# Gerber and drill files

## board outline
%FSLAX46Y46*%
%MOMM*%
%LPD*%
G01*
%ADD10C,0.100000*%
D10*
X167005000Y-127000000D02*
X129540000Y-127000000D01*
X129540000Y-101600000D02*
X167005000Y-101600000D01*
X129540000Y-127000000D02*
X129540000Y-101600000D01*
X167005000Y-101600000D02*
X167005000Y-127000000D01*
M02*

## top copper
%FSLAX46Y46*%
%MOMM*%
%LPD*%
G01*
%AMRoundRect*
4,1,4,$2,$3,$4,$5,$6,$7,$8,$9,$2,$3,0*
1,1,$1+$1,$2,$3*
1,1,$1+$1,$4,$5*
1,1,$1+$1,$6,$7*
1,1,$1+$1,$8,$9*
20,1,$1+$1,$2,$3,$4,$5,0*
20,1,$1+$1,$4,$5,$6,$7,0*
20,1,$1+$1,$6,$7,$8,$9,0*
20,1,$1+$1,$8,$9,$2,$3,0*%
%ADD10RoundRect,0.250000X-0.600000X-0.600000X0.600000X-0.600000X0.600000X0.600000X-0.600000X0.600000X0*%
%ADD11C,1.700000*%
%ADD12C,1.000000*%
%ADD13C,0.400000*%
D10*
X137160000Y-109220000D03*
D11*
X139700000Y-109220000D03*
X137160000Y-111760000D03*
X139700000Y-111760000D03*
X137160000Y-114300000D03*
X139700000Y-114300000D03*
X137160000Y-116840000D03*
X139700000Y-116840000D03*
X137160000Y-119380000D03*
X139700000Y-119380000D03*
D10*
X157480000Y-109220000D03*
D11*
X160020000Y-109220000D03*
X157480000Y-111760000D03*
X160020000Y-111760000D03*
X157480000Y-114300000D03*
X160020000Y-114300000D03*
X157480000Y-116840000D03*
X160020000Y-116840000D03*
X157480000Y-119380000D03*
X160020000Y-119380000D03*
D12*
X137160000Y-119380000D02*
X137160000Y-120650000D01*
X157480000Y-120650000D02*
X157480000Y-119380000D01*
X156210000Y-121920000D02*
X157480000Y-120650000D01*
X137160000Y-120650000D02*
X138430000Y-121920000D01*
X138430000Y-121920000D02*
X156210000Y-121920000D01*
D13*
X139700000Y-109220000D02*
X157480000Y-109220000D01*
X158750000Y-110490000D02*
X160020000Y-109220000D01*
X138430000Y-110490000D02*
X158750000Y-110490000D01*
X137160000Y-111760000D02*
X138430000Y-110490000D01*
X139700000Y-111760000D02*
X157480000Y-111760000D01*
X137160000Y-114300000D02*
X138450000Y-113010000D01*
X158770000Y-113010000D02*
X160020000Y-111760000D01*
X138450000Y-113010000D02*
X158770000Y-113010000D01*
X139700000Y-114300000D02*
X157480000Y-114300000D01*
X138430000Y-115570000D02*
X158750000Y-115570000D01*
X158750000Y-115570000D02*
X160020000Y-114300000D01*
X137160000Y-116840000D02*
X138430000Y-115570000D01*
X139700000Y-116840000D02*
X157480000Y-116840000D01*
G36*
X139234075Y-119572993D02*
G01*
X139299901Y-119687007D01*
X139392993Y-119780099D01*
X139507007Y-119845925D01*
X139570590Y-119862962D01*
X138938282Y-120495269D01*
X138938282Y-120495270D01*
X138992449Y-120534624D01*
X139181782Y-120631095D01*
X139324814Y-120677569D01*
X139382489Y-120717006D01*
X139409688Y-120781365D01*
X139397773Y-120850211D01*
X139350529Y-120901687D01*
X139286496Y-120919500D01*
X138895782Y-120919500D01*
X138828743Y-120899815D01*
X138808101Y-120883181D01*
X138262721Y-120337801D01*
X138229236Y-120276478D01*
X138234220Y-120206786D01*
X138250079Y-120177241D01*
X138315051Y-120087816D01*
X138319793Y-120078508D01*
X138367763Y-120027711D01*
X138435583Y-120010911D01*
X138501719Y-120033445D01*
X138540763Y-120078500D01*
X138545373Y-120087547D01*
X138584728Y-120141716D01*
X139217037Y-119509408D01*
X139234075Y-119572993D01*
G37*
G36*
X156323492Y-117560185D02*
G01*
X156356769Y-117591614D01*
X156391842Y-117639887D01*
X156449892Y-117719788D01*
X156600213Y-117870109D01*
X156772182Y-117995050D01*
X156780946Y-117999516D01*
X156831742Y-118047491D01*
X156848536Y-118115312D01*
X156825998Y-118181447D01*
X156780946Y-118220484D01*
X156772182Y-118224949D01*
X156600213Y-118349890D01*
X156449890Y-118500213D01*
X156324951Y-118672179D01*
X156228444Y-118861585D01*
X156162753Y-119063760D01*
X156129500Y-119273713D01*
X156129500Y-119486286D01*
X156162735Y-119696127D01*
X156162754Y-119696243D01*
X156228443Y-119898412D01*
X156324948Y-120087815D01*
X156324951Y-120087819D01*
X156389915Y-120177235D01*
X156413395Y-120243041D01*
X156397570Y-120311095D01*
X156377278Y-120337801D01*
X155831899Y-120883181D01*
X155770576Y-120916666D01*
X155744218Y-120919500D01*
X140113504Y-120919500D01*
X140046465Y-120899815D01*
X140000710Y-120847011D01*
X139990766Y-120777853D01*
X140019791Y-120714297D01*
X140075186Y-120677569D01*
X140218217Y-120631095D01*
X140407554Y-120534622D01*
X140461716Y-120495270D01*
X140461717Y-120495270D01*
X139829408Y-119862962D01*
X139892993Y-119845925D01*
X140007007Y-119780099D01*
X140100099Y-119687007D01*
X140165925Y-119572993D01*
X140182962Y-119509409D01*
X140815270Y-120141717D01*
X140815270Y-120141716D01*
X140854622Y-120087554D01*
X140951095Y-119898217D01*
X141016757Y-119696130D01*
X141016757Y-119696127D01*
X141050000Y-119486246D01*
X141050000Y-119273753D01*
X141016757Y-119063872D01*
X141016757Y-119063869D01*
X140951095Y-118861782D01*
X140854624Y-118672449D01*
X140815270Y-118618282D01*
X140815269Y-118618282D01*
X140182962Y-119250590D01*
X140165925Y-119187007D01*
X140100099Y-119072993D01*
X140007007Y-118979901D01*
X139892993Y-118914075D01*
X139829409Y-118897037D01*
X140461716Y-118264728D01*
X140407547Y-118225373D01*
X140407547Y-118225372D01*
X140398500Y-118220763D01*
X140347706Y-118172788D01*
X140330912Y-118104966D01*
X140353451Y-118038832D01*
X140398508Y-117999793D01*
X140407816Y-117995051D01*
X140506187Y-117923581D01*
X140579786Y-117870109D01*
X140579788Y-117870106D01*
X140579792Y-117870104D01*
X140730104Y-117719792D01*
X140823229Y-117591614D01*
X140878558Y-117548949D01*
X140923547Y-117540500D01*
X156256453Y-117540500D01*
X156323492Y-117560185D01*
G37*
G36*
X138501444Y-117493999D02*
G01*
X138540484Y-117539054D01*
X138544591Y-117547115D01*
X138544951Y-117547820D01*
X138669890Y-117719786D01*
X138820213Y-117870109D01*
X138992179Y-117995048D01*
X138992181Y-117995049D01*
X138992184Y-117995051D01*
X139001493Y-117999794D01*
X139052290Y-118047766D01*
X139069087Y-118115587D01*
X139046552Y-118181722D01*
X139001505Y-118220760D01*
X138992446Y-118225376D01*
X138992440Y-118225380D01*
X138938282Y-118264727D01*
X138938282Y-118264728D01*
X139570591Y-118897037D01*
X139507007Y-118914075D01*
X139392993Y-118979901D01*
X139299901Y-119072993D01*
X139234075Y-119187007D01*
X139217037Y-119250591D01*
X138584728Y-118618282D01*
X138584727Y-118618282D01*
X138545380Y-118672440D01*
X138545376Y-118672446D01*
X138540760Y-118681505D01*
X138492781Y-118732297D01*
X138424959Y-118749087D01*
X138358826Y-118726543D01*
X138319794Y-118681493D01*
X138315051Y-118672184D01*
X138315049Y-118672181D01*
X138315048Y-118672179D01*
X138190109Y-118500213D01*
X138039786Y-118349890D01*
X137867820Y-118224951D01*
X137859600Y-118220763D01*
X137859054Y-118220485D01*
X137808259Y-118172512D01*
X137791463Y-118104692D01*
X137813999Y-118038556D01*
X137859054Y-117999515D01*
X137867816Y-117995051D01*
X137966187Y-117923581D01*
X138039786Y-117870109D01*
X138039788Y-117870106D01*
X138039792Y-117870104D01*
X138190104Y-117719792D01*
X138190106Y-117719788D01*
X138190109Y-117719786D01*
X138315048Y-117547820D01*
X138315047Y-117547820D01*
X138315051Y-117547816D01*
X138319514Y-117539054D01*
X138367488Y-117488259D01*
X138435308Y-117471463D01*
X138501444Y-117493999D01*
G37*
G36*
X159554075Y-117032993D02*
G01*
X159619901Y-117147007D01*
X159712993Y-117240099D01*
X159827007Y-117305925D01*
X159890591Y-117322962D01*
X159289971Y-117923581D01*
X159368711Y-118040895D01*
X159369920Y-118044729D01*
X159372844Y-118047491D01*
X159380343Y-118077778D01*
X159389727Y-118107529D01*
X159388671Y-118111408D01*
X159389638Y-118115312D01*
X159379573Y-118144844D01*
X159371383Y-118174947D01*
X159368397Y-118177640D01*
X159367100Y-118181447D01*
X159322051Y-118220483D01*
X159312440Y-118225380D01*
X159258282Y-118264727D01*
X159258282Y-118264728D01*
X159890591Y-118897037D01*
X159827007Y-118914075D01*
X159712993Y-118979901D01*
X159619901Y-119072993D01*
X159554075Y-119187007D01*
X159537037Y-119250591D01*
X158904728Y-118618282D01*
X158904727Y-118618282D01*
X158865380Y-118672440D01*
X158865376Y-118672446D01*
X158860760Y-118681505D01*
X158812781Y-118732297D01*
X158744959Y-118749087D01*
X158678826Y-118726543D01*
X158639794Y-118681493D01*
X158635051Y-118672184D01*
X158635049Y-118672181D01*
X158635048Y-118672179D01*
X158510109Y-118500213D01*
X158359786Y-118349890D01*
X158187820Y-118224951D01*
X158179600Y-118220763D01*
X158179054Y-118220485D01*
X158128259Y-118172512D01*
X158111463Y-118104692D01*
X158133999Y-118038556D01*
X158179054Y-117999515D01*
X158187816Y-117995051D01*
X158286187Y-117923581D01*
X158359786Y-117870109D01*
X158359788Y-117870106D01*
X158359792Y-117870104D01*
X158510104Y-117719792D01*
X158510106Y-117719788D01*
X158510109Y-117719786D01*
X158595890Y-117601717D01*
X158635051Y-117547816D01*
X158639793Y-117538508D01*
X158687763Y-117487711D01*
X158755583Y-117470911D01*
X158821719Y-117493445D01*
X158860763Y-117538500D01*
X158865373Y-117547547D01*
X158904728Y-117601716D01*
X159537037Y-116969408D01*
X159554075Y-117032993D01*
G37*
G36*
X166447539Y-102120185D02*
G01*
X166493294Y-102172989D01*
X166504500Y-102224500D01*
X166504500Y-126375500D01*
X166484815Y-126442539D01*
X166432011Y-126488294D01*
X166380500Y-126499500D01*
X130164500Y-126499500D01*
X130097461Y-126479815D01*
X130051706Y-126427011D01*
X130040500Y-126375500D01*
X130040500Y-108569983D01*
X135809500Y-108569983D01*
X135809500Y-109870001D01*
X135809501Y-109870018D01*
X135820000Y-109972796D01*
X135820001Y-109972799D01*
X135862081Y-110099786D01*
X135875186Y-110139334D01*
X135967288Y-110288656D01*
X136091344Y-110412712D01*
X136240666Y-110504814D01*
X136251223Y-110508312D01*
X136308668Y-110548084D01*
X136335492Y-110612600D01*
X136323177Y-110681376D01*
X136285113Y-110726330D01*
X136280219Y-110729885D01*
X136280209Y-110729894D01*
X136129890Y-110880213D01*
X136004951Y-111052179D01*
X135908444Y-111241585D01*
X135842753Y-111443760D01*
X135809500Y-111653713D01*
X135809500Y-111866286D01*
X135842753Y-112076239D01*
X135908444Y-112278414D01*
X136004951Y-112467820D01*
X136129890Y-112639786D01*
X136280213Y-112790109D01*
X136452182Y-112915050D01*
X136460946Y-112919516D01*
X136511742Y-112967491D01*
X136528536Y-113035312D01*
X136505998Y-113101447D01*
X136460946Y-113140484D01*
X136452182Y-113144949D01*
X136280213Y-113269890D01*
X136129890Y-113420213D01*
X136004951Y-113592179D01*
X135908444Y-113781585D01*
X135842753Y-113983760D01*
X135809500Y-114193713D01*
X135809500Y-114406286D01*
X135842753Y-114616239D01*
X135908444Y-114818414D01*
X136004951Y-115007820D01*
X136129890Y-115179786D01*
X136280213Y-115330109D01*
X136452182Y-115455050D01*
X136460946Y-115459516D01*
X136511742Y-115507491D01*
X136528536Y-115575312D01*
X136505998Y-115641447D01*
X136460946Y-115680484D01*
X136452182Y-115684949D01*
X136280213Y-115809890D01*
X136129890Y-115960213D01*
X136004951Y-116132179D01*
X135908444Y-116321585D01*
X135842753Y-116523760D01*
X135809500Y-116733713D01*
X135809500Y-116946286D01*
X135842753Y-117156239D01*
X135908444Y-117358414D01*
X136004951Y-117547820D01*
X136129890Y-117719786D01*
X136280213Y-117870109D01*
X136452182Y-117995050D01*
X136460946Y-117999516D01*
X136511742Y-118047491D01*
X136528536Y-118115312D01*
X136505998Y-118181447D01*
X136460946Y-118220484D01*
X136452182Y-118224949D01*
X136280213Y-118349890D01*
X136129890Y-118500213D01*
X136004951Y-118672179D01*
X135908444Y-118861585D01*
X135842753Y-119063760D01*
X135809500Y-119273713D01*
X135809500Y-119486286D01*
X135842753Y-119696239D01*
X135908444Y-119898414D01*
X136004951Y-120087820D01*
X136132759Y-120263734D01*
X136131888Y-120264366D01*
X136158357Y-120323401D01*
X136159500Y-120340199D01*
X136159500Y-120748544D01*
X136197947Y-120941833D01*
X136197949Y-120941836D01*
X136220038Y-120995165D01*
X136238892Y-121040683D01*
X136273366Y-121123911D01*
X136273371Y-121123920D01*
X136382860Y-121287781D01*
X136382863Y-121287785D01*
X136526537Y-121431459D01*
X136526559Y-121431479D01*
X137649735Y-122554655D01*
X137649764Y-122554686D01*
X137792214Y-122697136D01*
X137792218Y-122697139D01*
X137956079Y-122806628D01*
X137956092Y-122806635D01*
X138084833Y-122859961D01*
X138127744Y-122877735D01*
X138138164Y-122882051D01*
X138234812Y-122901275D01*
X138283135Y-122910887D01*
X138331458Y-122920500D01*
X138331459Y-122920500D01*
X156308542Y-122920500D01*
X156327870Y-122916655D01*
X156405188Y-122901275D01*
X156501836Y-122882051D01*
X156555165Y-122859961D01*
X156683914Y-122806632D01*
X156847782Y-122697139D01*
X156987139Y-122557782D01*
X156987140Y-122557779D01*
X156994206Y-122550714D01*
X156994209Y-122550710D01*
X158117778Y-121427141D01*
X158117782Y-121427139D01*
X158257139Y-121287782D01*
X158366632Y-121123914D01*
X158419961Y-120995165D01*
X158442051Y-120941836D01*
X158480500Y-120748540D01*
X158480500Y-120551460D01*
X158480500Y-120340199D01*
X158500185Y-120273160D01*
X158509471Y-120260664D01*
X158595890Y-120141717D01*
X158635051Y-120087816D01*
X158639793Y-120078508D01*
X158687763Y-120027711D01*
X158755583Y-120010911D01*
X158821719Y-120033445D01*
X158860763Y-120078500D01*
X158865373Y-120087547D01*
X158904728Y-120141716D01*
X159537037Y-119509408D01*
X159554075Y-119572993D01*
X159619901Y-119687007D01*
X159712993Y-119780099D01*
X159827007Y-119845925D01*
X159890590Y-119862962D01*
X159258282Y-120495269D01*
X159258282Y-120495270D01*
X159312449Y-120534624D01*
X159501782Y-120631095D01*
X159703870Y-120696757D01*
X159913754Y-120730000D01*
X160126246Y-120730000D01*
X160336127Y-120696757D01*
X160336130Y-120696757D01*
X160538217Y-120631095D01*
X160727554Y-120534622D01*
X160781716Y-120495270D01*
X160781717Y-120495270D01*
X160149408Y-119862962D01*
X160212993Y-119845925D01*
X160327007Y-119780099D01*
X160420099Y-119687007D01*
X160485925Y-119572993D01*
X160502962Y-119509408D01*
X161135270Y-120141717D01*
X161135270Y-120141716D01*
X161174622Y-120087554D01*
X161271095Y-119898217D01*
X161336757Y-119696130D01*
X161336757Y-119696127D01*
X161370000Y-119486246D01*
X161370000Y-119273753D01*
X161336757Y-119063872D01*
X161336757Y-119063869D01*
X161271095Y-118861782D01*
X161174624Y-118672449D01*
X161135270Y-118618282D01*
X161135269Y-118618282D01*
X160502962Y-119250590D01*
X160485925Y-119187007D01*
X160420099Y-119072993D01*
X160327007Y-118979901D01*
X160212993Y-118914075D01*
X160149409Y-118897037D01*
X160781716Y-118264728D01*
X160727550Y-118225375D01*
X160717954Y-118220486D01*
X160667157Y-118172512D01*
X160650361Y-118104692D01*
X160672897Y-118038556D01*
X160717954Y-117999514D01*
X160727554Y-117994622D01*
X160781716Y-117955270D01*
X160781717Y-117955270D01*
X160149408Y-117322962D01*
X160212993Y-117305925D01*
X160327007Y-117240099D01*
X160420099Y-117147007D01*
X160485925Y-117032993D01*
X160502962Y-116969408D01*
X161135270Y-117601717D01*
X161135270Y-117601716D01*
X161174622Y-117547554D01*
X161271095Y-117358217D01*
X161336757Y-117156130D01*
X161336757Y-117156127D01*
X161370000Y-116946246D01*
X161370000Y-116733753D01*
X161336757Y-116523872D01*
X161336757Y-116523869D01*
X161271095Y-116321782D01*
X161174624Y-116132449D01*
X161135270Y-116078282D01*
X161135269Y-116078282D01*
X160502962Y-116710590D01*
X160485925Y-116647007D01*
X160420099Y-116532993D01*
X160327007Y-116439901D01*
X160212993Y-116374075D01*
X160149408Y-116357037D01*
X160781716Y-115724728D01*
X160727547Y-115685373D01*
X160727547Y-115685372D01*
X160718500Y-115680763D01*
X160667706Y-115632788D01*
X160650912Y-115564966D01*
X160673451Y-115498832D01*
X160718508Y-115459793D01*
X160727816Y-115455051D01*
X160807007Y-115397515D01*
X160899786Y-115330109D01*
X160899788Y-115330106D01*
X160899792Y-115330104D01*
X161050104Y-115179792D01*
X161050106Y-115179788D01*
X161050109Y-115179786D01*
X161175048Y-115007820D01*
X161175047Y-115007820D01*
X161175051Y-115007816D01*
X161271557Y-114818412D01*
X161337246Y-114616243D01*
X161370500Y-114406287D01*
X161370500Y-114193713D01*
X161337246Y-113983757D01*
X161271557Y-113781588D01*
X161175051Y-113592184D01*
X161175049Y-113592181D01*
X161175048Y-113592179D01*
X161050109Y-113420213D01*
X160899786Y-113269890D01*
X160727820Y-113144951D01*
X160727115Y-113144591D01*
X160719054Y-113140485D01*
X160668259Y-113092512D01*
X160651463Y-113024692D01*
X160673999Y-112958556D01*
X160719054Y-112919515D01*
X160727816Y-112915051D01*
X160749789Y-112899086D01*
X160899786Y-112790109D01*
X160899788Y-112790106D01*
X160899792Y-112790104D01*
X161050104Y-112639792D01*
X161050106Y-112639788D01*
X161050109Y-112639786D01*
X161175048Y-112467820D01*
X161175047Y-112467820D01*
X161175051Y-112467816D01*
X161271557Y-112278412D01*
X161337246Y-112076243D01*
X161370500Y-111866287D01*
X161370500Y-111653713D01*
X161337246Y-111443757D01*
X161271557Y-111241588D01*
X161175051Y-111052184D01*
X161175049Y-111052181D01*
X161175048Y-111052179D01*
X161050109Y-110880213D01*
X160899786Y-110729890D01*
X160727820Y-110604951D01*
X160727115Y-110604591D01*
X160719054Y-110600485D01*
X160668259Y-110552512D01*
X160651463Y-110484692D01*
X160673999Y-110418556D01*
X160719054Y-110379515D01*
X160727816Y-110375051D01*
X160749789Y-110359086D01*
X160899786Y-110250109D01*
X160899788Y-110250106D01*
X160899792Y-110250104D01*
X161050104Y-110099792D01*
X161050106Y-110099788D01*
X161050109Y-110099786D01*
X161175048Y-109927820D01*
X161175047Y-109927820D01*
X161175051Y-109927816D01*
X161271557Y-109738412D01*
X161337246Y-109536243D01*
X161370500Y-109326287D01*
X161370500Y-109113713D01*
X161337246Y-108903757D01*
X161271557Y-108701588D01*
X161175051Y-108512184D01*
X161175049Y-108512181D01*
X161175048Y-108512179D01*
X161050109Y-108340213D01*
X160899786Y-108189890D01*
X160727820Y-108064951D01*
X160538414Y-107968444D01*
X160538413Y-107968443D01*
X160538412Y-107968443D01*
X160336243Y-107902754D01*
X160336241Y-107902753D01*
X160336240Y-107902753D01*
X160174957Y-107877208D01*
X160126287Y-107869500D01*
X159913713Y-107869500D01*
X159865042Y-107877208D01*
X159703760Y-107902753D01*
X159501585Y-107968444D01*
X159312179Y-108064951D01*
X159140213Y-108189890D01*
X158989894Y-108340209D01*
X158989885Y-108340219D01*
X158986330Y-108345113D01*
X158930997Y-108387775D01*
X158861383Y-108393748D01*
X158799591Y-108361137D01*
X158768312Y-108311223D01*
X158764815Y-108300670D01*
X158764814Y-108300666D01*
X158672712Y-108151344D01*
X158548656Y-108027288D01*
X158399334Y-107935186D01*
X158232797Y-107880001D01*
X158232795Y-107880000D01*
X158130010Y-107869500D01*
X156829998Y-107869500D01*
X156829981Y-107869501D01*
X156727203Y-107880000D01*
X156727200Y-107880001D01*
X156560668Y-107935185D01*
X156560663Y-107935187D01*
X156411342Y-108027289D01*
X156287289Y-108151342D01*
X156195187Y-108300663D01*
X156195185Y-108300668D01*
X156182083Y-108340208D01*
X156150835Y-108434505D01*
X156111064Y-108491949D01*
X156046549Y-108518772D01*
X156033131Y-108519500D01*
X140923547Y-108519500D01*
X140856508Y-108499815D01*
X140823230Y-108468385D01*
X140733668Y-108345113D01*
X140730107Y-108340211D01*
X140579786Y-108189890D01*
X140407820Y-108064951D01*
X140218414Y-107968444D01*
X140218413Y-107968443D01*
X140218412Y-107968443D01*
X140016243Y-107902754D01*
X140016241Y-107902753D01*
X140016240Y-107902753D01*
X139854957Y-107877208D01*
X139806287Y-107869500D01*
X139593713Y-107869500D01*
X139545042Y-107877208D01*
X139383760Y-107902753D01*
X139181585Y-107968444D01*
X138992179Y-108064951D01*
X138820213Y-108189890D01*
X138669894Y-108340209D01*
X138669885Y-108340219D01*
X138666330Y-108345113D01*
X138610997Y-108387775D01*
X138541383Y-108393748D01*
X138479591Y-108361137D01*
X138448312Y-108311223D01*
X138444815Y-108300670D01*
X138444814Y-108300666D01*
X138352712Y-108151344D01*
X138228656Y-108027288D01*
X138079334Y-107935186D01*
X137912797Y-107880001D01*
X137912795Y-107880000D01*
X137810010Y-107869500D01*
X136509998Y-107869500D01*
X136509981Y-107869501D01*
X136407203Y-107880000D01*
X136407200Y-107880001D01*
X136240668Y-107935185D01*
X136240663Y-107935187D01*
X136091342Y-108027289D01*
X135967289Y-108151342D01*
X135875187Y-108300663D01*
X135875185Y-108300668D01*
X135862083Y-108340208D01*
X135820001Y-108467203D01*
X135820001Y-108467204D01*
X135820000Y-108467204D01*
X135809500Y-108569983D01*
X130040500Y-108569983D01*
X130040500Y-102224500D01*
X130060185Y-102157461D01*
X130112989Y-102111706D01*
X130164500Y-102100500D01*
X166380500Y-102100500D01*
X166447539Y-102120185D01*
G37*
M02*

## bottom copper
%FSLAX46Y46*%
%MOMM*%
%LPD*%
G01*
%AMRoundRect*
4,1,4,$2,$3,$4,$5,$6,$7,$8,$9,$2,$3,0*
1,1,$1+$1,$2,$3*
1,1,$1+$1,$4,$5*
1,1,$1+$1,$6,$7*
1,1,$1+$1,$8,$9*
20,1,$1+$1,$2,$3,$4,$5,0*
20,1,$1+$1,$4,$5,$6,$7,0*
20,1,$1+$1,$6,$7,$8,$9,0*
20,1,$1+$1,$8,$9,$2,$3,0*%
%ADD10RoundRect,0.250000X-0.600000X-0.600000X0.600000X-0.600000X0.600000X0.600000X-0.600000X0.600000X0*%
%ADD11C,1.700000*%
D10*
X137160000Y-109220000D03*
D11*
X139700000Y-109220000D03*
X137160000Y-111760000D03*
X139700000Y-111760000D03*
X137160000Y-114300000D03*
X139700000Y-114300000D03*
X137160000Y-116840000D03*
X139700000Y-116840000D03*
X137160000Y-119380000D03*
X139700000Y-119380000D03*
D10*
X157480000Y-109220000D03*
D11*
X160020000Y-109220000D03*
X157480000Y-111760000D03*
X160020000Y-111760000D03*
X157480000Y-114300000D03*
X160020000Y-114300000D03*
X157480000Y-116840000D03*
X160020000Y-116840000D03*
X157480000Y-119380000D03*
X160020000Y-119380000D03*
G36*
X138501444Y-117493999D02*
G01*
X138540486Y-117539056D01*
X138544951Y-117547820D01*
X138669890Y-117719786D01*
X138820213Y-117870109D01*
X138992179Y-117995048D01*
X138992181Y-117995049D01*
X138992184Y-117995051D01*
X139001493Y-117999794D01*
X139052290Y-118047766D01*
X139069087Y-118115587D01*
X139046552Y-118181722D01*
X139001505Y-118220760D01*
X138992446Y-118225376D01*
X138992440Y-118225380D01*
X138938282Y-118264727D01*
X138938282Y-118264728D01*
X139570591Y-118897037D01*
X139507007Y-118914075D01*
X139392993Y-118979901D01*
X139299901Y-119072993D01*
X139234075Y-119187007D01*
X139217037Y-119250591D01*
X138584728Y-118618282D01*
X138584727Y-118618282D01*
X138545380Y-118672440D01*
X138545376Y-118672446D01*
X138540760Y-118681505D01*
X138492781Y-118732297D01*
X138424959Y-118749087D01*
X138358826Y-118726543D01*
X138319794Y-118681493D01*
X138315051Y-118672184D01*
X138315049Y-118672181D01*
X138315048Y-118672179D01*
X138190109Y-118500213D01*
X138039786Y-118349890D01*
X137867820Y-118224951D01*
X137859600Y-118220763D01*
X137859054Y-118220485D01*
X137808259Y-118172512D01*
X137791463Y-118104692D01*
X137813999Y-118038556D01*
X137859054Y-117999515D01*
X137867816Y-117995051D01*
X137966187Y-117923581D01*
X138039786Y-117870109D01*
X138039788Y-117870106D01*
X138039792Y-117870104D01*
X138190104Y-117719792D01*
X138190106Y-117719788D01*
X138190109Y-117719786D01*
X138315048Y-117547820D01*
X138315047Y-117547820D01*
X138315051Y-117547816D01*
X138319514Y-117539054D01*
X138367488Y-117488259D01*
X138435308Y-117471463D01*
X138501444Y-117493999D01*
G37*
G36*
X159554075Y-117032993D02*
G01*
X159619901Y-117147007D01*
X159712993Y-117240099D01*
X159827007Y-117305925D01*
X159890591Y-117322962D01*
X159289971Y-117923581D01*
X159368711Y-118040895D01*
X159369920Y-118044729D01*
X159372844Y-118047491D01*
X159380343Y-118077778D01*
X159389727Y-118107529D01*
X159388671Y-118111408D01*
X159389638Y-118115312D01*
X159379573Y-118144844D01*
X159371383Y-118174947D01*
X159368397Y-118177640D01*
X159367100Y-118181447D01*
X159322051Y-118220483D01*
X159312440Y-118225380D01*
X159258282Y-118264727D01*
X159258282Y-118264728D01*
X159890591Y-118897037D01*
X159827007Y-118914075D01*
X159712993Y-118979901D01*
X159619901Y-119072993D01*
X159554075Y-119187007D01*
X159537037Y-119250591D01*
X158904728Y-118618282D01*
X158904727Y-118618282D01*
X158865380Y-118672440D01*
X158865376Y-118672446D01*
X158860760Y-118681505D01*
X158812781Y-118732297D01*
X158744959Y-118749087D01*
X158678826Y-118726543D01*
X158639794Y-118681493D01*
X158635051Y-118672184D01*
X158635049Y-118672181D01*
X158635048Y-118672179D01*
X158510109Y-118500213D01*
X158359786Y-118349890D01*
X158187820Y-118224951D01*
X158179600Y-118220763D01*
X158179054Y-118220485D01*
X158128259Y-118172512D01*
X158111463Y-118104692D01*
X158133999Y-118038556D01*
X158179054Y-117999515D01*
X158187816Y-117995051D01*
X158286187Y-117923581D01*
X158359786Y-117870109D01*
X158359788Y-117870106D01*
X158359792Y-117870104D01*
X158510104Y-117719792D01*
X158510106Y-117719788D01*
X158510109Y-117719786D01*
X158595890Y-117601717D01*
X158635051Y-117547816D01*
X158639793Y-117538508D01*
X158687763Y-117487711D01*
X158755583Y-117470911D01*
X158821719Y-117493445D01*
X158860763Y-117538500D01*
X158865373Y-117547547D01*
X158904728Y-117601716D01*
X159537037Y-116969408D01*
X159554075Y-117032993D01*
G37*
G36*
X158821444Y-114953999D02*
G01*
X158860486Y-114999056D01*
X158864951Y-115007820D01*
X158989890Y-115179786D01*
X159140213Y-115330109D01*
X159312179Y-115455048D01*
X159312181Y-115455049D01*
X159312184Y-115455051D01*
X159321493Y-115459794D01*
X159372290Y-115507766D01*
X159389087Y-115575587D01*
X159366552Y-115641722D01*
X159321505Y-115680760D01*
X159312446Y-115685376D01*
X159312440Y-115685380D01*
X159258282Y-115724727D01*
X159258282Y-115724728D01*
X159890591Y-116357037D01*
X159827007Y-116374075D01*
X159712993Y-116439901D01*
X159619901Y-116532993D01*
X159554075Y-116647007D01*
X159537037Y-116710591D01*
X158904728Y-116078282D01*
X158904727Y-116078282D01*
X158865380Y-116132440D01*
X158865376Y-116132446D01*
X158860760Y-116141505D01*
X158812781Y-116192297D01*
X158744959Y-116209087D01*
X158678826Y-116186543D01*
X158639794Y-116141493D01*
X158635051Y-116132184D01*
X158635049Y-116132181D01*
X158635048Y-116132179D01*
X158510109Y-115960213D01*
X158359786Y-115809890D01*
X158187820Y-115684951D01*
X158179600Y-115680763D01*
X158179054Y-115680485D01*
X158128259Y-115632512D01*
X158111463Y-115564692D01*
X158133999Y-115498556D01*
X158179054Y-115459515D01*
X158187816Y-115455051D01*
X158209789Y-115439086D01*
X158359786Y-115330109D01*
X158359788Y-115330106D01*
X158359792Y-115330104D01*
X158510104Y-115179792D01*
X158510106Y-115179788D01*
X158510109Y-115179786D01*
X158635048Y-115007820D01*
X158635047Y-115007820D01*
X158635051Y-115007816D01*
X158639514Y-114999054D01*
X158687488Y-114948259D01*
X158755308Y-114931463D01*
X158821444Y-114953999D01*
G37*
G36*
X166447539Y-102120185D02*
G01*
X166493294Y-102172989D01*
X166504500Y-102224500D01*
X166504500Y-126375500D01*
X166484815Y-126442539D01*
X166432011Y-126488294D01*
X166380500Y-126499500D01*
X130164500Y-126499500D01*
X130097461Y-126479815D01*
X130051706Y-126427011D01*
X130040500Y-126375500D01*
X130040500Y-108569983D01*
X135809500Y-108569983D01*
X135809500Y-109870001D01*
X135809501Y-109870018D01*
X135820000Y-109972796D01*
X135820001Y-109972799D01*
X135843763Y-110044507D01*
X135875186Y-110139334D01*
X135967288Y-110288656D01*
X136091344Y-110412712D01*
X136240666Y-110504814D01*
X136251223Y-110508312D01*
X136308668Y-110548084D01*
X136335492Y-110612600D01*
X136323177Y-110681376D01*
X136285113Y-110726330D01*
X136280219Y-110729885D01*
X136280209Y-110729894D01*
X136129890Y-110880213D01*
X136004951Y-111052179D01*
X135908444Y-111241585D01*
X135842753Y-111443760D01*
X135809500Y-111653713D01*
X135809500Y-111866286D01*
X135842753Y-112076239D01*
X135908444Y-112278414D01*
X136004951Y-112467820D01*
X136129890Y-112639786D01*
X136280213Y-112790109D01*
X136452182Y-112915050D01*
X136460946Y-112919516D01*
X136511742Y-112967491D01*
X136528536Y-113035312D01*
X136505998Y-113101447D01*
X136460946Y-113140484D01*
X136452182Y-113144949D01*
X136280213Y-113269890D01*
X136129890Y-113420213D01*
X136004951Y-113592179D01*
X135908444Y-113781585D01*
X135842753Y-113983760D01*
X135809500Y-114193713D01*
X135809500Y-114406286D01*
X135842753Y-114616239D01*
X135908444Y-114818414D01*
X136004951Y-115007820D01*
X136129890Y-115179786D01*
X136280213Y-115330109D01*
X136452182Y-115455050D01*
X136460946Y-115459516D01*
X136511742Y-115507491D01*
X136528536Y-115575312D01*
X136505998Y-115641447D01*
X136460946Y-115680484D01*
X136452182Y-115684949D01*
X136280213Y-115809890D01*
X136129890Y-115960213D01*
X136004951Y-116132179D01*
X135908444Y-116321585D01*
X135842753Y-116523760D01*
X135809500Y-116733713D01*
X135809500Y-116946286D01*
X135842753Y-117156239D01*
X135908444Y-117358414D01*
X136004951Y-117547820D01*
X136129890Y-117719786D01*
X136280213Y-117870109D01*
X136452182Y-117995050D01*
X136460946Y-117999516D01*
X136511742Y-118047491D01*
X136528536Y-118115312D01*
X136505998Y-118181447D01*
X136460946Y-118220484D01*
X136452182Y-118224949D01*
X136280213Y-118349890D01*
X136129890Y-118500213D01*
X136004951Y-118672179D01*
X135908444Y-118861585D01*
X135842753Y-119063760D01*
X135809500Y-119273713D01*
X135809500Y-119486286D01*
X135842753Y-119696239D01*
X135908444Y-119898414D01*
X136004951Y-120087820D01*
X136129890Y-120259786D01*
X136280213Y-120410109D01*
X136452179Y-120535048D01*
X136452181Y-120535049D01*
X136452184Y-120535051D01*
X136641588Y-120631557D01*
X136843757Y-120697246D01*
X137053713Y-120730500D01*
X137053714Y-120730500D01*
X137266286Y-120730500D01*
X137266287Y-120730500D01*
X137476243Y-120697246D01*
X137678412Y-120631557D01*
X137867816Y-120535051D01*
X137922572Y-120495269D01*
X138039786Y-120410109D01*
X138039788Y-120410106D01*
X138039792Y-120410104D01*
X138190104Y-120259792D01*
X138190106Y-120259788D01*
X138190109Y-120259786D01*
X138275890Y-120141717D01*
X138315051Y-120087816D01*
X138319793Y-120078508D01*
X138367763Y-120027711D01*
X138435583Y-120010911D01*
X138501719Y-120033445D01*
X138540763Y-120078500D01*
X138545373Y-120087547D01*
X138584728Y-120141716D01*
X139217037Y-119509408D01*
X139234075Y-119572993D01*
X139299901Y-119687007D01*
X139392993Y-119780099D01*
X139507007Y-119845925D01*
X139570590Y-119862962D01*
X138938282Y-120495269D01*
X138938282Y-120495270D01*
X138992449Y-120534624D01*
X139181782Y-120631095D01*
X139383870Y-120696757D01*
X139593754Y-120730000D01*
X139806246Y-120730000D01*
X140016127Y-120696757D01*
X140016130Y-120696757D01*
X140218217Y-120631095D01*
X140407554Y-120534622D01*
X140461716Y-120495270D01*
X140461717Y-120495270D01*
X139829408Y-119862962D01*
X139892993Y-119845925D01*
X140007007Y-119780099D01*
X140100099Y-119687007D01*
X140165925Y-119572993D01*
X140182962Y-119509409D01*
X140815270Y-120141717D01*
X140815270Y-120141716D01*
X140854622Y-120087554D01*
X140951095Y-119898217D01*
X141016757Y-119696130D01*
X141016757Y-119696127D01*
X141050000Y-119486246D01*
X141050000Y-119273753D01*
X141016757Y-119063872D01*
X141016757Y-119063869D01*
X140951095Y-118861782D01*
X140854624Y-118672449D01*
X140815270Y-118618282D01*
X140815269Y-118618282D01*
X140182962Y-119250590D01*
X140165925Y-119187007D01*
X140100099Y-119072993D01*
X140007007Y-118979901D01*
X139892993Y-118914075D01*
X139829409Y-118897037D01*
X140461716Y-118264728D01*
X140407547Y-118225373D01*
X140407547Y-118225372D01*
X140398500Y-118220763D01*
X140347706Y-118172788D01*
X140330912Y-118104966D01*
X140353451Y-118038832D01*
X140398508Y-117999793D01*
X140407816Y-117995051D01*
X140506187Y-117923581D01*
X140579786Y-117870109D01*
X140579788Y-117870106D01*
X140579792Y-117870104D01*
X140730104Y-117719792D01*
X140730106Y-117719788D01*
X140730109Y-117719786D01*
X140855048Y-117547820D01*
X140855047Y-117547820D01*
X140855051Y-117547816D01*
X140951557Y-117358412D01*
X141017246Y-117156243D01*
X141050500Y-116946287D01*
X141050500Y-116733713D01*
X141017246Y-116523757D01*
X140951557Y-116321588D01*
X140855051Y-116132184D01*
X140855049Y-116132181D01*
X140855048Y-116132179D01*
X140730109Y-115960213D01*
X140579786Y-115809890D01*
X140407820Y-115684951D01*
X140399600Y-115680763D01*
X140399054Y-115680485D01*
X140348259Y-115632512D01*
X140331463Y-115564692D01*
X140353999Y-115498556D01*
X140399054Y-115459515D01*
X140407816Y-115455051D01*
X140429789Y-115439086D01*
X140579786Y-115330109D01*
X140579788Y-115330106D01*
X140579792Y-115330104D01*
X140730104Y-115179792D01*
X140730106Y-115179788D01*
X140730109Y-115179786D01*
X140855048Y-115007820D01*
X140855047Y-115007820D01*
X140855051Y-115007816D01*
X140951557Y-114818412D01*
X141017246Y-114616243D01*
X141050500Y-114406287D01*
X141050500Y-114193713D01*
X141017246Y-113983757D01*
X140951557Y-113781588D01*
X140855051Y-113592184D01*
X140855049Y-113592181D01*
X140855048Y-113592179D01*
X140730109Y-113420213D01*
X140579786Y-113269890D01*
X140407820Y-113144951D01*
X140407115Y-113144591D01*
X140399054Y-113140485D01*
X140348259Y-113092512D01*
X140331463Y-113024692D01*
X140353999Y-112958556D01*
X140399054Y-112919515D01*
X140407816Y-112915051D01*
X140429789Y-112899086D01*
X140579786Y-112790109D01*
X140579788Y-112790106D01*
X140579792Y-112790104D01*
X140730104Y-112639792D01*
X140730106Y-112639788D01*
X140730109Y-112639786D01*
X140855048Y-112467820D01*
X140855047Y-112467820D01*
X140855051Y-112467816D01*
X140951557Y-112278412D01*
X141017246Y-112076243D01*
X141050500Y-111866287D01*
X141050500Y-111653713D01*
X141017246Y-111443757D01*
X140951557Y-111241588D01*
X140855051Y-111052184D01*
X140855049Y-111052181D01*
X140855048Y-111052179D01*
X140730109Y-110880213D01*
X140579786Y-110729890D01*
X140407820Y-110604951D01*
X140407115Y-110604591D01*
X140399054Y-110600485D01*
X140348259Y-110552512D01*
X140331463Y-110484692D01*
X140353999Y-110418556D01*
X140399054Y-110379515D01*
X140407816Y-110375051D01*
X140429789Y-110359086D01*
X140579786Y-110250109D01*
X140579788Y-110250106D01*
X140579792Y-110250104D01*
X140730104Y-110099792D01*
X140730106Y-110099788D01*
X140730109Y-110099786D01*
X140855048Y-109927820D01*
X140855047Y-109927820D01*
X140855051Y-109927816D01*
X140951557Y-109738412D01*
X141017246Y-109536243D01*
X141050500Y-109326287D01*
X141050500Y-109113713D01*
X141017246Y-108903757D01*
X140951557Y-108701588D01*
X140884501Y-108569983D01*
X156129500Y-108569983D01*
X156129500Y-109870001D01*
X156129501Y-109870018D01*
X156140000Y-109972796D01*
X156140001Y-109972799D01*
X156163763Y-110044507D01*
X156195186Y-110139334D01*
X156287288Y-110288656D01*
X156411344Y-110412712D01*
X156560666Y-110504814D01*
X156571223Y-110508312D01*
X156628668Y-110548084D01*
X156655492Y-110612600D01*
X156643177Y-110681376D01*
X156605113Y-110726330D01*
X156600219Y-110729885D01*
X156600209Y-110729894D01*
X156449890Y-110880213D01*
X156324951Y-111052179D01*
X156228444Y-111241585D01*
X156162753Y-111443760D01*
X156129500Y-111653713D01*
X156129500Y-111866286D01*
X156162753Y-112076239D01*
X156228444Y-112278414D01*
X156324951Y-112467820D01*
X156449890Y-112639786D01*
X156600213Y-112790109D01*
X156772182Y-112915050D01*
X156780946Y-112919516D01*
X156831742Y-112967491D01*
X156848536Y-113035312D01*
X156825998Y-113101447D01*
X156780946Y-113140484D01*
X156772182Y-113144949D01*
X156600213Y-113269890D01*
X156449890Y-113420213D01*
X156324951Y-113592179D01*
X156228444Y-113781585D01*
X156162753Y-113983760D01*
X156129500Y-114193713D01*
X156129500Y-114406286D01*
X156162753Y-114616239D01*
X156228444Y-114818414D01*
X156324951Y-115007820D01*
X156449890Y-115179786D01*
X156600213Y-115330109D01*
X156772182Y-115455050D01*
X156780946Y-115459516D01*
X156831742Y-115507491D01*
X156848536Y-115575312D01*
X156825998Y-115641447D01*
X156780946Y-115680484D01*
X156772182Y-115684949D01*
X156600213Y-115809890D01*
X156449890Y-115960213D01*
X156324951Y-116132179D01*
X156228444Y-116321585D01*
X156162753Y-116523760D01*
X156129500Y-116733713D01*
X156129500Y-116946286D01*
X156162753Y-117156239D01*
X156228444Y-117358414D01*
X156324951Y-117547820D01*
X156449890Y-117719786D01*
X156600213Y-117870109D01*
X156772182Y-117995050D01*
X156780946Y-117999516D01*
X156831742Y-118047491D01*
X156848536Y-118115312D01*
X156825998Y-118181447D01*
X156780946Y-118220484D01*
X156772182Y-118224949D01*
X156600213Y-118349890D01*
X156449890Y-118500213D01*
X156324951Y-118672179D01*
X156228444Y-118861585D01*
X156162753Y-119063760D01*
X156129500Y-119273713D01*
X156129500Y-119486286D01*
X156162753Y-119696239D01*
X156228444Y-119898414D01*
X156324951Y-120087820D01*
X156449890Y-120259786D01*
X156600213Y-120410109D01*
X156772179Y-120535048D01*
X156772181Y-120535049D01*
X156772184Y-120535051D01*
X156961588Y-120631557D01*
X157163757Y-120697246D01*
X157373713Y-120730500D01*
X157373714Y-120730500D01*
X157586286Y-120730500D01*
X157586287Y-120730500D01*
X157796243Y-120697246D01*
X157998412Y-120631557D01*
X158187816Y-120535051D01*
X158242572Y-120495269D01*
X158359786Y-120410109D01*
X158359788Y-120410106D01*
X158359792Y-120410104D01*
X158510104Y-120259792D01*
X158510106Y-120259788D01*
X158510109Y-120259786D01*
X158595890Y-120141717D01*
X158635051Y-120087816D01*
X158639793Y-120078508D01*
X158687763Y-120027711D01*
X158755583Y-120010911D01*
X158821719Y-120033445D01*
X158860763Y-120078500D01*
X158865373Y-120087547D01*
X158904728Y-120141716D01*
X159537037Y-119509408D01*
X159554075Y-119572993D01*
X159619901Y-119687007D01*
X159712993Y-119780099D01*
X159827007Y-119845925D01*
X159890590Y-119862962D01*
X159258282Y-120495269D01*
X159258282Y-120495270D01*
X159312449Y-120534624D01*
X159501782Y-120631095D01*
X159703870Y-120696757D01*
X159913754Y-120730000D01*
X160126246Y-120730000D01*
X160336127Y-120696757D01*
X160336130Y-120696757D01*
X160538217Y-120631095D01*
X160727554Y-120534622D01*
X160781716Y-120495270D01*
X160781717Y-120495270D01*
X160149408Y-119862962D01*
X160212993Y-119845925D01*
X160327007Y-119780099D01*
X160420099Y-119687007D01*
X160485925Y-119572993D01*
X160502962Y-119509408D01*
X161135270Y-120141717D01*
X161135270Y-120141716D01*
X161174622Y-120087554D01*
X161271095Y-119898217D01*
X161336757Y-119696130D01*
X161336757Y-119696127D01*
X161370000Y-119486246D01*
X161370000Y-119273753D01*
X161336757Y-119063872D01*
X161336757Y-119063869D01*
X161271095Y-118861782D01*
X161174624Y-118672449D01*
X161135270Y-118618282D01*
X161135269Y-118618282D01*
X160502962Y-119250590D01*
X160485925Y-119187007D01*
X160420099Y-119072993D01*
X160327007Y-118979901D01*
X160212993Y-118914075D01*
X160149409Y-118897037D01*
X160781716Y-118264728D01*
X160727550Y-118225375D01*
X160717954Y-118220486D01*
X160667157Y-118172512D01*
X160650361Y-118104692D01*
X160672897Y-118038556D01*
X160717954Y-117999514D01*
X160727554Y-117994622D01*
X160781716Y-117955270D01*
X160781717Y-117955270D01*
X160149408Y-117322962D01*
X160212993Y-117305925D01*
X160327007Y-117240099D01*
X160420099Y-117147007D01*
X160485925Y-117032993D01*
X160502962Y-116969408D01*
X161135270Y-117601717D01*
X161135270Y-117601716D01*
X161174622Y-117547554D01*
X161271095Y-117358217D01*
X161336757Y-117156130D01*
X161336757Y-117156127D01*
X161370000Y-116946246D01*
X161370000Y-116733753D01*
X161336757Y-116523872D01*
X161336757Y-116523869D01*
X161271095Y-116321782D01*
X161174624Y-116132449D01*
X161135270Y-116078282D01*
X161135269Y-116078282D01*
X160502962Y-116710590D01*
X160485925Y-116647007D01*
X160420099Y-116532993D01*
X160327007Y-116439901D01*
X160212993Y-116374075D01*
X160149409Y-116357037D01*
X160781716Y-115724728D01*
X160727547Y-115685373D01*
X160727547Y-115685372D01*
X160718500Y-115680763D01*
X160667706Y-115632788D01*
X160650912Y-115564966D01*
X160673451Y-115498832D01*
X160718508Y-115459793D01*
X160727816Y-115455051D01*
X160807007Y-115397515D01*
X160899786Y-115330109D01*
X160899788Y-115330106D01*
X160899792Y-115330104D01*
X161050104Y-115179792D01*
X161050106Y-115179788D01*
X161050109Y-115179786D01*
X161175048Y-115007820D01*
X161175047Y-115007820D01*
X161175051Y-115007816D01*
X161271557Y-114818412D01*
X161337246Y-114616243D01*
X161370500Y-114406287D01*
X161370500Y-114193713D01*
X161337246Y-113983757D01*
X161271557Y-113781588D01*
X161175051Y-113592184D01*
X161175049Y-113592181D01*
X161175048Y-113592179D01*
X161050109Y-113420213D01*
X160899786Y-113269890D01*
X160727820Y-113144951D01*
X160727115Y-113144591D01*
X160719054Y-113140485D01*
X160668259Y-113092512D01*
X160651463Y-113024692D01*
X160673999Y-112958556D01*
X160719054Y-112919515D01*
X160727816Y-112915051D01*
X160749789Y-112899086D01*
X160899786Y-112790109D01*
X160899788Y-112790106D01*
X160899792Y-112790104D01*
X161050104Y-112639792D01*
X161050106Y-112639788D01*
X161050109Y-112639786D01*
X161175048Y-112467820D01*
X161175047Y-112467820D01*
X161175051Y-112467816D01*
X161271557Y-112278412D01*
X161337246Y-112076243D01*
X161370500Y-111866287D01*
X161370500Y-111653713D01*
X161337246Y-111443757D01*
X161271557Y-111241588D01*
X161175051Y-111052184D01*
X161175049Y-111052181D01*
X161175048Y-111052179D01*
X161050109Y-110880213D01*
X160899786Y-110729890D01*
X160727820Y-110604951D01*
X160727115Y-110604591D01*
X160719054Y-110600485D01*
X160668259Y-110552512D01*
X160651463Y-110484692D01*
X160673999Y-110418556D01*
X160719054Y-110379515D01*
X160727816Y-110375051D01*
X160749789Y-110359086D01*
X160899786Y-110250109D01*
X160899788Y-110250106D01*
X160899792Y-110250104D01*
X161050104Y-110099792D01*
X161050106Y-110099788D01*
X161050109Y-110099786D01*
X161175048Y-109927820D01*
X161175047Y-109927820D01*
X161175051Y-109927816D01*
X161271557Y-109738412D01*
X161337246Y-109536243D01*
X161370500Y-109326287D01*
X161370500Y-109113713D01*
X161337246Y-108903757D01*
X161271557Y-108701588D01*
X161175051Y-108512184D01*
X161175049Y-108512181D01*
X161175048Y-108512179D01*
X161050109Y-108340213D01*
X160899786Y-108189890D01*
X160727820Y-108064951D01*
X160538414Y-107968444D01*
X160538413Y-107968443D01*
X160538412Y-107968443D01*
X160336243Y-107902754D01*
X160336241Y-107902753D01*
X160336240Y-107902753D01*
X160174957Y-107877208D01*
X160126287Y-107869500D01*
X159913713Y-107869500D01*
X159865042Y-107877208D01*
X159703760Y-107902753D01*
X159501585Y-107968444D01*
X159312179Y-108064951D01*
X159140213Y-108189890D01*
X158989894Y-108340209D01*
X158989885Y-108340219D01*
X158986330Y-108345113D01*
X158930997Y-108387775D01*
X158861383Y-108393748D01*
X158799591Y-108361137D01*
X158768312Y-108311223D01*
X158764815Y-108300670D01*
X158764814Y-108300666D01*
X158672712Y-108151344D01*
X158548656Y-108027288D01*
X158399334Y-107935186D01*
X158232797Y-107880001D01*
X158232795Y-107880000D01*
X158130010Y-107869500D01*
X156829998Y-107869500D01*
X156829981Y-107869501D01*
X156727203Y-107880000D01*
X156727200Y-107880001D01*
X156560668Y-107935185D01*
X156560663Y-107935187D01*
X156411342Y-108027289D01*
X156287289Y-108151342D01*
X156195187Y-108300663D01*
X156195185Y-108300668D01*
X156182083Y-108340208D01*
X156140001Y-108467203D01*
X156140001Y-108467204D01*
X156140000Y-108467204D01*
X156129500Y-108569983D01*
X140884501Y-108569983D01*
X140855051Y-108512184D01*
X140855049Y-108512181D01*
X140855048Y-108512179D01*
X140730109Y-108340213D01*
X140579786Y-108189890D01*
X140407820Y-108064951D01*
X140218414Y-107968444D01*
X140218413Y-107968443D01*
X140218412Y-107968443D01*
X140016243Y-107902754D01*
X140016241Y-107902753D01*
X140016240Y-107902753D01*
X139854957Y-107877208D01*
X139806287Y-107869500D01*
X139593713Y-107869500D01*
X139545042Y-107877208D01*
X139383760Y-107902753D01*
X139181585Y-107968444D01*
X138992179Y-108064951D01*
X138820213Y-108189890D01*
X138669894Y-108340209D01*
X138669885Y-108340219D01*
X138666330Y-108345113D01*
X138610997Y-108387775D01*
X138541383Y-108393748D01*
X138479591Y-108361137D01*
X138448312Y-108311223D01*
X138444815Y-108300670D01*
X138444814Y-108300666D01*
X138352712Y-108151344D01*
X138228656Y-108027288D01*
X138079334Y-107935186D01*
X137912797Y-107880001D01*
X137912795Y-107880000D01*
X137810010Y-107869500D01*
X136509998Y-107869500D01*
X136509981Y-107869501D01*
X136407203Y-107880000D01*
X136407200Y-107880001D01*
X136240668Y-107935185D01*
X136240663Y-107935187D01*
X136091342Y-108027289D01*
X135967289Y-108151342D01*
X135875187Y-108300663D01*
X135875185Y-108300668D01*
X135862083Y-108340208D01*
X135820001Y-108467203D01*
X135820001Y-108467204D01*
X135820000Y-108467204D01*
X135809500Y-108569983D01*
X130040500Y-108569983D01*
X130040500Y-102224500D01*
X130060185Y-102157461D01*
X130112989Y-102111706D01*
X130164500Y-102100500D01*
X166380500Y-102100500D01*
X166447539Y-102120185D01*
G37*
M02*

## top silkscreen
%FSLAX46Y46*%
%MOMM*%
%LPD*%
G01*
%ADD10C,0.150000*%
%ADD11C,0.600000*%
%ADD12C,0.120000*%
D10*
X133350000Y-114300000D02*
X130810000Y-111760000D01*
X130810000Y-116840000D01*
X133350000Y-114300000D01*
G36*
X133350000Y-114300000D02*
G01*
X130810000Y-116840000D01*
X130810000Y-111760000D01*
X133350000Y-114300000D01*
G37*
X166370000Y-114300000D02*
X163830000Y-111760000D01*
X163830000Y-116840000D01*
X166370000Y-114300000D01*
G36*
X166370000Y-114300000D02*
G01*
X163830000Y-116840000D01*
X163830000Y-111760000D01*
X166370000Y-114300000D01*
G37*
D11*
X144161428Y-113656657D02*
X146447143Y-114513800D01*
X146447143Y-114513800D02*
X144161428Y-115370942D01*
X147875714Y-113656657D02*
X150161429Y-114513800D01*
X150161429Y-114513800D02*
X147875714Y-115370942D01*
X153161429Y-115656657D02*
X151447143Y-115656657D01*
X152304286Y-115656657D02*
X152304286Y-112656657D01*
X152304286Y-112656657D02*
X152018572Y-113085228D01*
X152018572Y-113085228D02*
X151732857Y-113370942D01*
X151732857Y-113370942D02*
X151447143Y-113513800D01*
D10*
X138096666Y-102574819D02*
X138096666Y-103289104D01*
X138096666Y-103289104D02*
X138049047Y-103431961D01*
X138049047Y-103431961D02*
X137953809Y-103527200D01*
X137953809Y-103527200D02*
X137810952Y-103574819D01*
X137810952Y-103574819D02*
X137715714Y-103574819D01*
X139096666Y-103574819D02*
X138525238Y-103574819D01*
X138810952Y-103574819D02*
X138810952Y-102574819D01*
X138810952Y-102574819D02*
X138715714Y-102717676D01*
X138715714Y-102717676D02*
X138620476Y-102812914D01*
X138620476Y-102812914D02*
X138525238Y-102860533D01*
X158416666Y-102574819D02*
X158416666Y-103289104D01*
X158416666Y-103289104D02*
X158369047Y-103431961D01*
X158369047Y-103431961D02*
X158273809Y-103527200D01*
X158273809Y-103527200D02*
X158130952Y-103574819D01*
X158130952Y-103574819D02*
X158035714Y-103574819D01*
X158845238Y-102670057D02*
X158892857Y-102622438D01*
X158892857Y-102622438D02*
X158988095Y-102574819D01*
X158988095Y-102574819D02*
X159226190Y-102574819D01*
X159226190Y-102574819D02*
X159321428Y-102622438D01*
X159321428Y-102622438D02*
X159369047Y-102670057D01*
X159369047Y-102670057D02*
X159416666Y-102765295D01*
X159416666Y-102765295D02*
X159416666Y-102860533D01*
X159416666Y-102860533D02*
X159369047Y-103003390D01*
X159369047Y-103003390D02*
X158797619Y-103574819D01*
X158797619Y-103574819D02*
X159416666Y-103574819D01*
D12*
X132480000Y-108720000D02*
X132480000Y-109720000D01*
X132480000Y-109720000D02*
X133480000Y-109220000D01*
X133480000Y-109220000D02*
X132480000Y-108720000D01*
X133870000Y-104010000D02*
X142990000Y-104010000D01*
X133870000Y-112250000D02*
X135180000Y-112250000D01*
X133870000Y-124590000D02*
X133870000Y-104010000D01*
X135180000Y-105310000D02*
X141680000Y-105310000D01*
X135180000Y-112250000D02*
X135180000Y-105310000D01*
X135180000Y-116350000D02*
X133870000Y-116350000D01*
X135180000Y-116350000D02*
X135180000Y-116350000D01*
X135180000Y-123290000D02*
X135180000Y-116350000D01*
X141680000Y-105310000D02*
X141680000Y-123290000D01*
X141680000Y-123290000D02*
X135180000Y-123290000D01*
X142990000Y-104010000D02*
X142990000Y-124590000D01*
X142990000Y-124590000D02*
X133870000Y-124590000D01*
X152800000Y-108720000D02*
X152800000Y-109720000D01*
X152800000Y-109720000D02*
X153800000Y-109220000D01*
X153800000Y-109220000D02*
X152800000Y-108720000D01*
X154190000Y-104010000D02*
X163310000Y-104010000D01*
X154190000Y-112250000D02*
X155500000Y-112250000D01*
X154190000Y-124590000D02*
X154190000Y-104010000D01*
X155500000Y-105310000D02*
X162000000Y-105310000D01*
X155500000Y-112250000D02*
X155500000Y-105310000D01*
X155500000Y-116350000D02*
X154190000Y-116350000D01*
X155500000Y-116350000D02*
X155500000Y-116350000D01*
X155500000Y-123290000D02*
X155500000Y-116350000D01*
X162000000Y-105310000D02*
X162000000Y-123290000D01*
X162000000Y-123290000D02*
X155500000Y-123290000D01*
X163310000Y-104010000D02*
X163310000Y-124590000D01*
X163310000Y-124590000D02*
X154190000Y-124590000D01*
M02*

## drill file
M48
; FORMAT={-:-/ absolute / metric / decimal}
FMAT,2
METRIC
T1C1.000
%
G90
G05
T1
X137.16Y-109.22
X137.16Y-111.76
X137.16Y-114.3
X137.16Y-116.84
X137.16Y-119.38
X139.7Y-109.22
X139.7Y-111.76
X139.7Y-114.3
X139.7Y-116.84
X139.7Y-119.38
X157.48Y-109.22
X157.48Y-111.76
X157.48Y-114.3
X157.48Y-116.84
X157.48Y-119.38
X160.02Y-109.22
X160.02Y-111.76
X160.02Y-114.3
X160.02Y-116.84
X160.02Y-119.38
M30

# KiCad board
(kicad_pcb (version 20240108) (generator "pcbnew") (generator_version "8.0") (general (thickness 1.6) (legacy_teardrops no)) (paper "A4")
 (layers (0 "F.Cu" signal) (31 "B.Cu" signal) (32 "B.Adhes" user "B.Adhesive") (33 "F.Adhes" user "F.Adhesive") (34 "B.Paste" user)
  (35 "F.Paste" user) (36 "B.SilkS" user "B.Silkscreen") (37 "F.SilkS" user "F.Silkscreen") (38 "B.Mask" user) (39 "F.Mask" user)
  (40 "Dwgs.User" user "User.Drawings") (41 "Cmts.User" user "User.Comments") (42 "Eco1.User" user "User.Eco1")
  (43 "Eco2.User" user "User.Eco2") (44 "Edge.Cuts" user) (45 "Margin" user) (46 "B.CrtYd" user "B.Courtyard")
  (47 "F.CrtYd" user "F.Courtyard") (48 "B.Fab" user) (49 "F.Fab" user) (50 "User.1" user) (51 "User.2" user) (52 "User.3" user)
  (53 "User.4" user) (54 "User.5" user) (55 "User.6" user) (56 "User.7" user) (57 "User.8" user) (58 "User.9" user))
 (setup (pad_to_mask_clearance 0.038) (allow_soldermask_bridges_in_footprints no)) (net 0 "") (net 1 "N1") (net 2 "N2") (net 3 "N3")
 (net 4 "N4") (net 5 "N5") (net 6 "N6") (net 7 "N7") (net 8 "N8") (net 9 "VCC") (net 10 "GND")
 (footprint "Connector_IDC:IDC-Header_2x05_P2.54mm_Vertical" (layer "F.Cu") (at 137.16 109.22)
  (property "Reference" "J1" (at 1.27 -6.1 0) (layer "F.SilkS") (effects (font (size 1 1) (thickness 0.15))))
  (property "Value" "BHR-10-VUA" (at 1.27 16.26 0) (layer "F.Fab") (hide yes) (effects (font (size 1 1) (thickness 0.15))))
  (fp_line (start -4.68 -0.5) (end -4.68 0.5) (stroke (width 0.12) (type solid)) (layer "F.SilkS"))
  (fp_line (start -4.68 0.5) (end -3.68 0) (stroke (width 0.12) (type solid)) (layer "F.SilkS"))
  (fp_line (start -3.68 0) (end -4.68 -0.5) (stroke (width 0.12) (type solid)) (layer "F.SilkS"))
  (fp_line (start -3.29 -5.21) (end 5.83 -5.21) (stroke (width 0.12) (type solid)) (layer "F.SilkS"))
  (fp_line (start -3.29 3.03) (end -1.98 3.03) (stroke (width 0.12) (type solid)) (layer "F.SilkS"))
  (fp_line (start -3.29 15.37) (end -3.29 -5.21) (stroke (width 0.12) (type solid)) (layer "F.SilkS"))
  (fp_line (start -1.98 -3.91) (end 4.52 -3.91) (stroke (width 0.12) (type solid)) (layer "F.SilkS"))
  (fp_line (start -1.98 3.03) (end -1.98 -3.91) (stroke (width 0.12) (type solid)) (layer "F.SilkS"))
  (fp_line (start -1.98 7.13) (end -3.29 7.13) (stroke (width 0.12) (type solid)) (layer "F.SilkS"))
  (fp_line (start -1.98 7.13) (end -1.98 7.13) (stroke (width 0.12) (type solid)) (layer "F.SilkS"))
  (fp_line (start -1.98 14.07) (end -1.98 7.13) (stroke (width 0.12) (type solid)) (layer "F.SilkS"))
  (fp_line (start 4.52 -3.91) (end 4.52 14.07) (stroke (width 0.12) (type solid)) (layer "F.SilkS"))
  (fp_line (start 4.52 14.07) (end -1.98 14.07) (stroke (width 0.12) (type solid)) (layer "F.SilkS"))
  (fp_line (start 5.83 -5.21) (end 5.83 15.37) (stroke (width 0.12) (type solid)) (layer "F.SilkS"))
  (fp_line (start 5.83 15.37) (end -3.29 15.37) (stroke (width 0.12) (type solid)) (layer "F.SilkS"))
  (pad "1" thru_hole roundrect (at 0 0) (size 1.7 1.7) (drill 1) (layers "*.Cu" "*.Mask") (remove_unused_layers no)
   (roundrect_rratio 0.147059) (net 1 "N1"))
  (pad "2" thru_hole circle (at 2.54 0) (size 1.7 1.7) (drill 1) (layers "*.Cu" "*.Mask") (remove_unused_layers no) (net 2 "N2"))
  (pad "3" thru_hole circle (at 0 2.54) (size 1.7 1.7) (drill 1) (layers "*.Cu" "*.Mask") (remove_unused_layers no) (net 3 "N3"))
  (pad "4" thru_hole circle (at 2.54 2.54) (size 1.7 1.7) (drill 1) (layers "*.Cu" "*.Mask") (remove_unused_layers no) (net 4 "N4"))
  (pad "5" thru_hole circle (at 0 5.08) (size 1.7 1.7) (drill 1) (layers "*.Cu" "*.Mask") (remove_unused_layers no) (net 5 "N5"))
  (pad "6" thru_hole circle (at 2.54 5.08) (size 1.7 1.7) (drill 1) (layers "*.Cu" "*.Mask") (remove_unused_layers no) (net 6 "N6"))
  (pad "7" thru_hole circle (at 0 7.62) (size 1.7 1.7) (drill 1) (layers "*.Cu" "*.Mask") (remove_unused_layers no) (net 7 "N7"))
  (pad "8" thru_hole circle (at 2.54 7.62) (size 1.7 1.7) (drill 1) (layers "*.Cu" "*.Mask") (remove_unused_layers no) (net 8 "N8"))
  (pad "9" thru_hole circle (at 0 10.16) (size 1.7 1.7) (drill 1) (layers "*.Cu" "*.Mask") (remove_unused_layers no) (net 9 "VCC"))
  (pad "10" thru_hole circle (at 2.54 10.16) (size 1.7 1.7) (drill 1) (layers "*.Cu" "*.Mask") (remove_unused_layers no) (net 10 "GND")))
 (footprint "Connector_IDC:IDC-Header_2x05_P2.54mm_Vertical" (layer "F.Cu") (at 157.48 109.22)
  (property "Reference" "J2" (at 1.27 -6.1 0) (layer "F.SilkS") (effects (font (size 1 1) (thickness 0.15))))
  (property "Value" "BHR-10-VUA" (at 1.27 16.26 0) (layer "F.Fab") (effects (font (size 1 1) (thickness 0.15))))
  (fp_line (start -4.68 -0.5) (end -4.68 0.5) (stroke (width 0.12) (type solid)) (layer "F.SilkS"))
  (fp_line (start -4.68 0.5) (end -3.68 0) (stroke (width 0.12) (type solid)) (layer "F.SilkS"))
  (fp_line (start -3.68 0) (end -4.68 -0.5) (stroke (width 0.12) (type solid)) (layer "F.SilkS"))
  (fp_line (start -3.29 -5.21) (end 5.83 -5.21) (stroke (width 0.12) (type solid)) (layer "F.SilkS"))
  (fp_line (start -3.29 3.03) (end -1.98 3.03) (stroke (width 0.12) (type solid)) (layer "F.SilkS"))
  (fp_line (start -3.29 15.37) (end -3.29 -5.21) (stroke (width 0.12) (type solid)) (layer "F.SilkS"))
  (fp_line (start -1.98 -3.91) (end 4.52 -3.91) (stroke (width 0.12) (type solid)) (layer "F.SilkS"))
  (fp_line (start -1.98 3.03) (end -1.98 -3.91) (stroke (width 0.12) (type solid)) (layer "F.SilkS"))
  (fp_line (start -1.98 7.13) (end -3.29 7.13) (stroke (width 0.12) (type solid)) (layer "F.SilkS"))
  (fp_line (start -1.98 7.13) (end -1.98 7.13) (stroke (width 0.12) (type solid)) (layer "F.SilkS"))
  (fp_line (start -1.98 14.07) (end -1.98 7.13) (stroke (width 0.12) (type solid)) (layer "F.SilkS"))
  (fp_line (start 4.52 -3.91) (end 4.52 14.07) (stroke (width 0.12) (type solid)) (layer "F.SilkS"))
  (fp_line (start 4.52 14.07) (end -1.98 14.07) (stroke (width 0.12) (type solid)) (layer "F.SilkS"))
  (fp_line (start 5.83 -5.21) (end 5.83 15.37) (stroke (width 0.12) (type solid)) (layer "F.SilkS"))
  (fp_line (start 5.83 15.37) (end -3.29 15.37) (stroke (width 0.12) (type solid)) (layer "F.SilkS"))
  (pad "1" thru_hole roundrect (at 0 0) (size 1.7 1.7) (drill 1) (layers "*.Cu" "*.Mask") (remove_unused_layers no)
   (roundrect_rratio 0.147059) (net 2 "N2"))
  (pad "2" thru_hole circle (at 2.54 0) (size 1.7 1.7) (drill 1) (layers "*.Cu" "*.Mask") (remove_unused_layers no) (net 3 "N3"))
  (pad "3" thru_hole circle (at 0 2.54) (size 1.7 1.7) (drill 1) (layers "*.Cu" "*.Mask") (remove_unused_layers no) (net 4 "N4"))
  (pad "4" thru_hole circle (at 2.54 2.54) (size 1.7 1.7) (drill 1) (layers "*.Cu" "*.Mask") (remove_unused_layers no) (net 5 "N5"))
  (pad "5" thru_hole circle (at 0 5.08) (size 1.7 1.7) (drill 1) (layers "*.Cu" "*.Mask") (remove_unused_layers no) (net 6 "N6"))
  (pad "6" thru_hole circle (at 2.54 5.08) (size 1.7 1.7) (drill 1) (layers "*.Cu" "*.Mask") (remove_unused_layers no) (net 7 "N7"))
  (pad "7" thru_hole circle (at 0 7.62) (size 1.7 1.7) (drill 1) (layers "*.Cu" "*.Mask") (remove_unused_layers no) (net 8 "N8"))
  (pad "8" thru_hole circle (at 2.54 7.62) (size 1.7 1.7) (drill 1) (layers "*.Cu" "*.Mask") (remove_unused_layers no) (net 10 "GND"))
  (pad "9" thru_hole circle (at 0 10.16) (size 1.7 1.7) (drill 1) (layers "*.Cu" "*.Mask") (remove_unused_layers no) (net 9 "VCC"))
  (pad "10" thru_hole circle (at 2.54 10.16) (size 1.7 1.7) (drill 1) (layers "*.Cu" "*.Mask") (remove_unused_layers no) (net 10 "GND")))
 (gr_poly (pts (xy 133.35 114.3) (xy 130.81 111.76) (xy 130.81 116.84)) (stroke (width 0.15) (type solid)) (fill solid) (layer "F.SilkS"))
 (gr_poly (pts (xy 166.37 114.3) (xy 163.83 111.76) (xy 163.83 116.84)) (stroke (width 0.15) (type solid)) (fill solid) (layer "F.SilkS"))
 (gr_line (start 167.005 127) (end 129.54 127) (stroke (width 0.1) (type default)) (layer "Edge.Cuts"))
 (gr_line (start 129.54 101.6) (end 167.005 101.6) (stroke (width 0.1) (type default)) (layer "Edge.Cuts"))
 (gr_line (start 129.54 127) (end 129.54 101.6) (stroke (width 0.1) (type default)) (layer "Edge.Cuts"))
 (gr_line (start 167.005 101.6) (end 167.005 127) (stroke (width 0.1) (type default)) (layer "Edge.Cuts"))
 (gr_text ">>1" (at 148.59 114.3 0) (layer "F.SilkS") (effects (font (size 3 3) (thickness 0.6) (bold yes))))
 (segment (start 137.16 119.38) (end 137.16 120.65) (width 1) (layer "F.Cu") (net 9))
 (segment (start 157.48 120.65) (end 157.48 119.38) (width 1) (layer "F.Cu") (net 9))
 (segment (start 156.21 121.92) (end 157.48 120.65) (width 1) (layer "F.Cu") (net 9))
 (segment (start 137.16 120.65) (end 138.43 121.92) (width 1) (layer "F.Cu") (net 9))
 (segment (start 138.43 121.92) (end 156.21 121.92) (width 1) (layer "F.Cu") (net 9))
 (segment (start 139.7 109.22) (end 157.48 109.22) (width 0.4) (layer "F.Cu") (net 2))
 (segment (start 158.75 110.49) (end 160.02 109.22) (width 0.4) (layer "F.Cu") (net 3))
 (segment (start 138.43 110.49) (end 158.75 110.49) (width 0.4) (layer "F.Cu") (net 3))
 (segment (start 137.16 111.76) (end 138.43 110.49) (width 0.4) (layer "F.Cu") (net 3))
 (segment (start 139.7 111.76) (end 157.48 111.76) (width 0.4) (layer "F.Cu") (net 4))
 (segment (start 137.16 114.3) (end 138.45 113.01) (width 0.4) (layer "F.Cu") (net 5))
 (segment (start 158.77 113.01) (end 160.02 111.76) (width 0.4) (layer "F.Cu") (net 5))
 (segment (start 138.45 113.01) (end 158.77 113.01) (width 0.4) (layer "F.Cu") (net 5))
 (segment (start 139.7 114.3) (end 157.48 114.3) (width 0.4) (layer "F.Cu") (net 6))
 (segment (start 138.43 115.57) (end 158.75 115.57) (width 0.4) (layer "F.Cu") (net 7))
 (segment (start 158.75 115.57) (end 160.02 114.3) (width 0.4) (layer "F.Cu") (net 7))
 (segment (start 137.16 116.84) (end 138.43 115.57) (width 0.4) (layer "F.Cu") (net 7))
 (segment (start 139.7 116.84) (end 157.48 116.84) (width 0.4) (layer "F.Cu") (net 8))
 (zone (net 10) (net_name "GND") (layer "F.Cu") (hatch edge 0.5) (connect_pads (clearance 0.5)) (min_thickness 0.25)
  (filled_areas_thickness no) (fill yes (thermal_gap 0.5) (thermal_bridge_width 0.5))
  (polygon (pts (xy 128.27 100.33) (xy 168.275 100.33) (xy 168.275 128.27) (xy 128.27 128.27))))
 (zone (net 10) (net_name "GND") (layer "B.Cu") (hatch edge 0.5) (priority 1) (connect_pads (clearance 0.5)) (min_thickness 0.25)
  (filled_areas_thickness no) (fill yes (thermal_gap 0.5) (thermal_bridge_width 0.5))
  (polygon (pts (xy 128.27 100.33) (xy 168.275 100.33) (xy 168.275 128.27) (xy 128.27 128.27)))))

